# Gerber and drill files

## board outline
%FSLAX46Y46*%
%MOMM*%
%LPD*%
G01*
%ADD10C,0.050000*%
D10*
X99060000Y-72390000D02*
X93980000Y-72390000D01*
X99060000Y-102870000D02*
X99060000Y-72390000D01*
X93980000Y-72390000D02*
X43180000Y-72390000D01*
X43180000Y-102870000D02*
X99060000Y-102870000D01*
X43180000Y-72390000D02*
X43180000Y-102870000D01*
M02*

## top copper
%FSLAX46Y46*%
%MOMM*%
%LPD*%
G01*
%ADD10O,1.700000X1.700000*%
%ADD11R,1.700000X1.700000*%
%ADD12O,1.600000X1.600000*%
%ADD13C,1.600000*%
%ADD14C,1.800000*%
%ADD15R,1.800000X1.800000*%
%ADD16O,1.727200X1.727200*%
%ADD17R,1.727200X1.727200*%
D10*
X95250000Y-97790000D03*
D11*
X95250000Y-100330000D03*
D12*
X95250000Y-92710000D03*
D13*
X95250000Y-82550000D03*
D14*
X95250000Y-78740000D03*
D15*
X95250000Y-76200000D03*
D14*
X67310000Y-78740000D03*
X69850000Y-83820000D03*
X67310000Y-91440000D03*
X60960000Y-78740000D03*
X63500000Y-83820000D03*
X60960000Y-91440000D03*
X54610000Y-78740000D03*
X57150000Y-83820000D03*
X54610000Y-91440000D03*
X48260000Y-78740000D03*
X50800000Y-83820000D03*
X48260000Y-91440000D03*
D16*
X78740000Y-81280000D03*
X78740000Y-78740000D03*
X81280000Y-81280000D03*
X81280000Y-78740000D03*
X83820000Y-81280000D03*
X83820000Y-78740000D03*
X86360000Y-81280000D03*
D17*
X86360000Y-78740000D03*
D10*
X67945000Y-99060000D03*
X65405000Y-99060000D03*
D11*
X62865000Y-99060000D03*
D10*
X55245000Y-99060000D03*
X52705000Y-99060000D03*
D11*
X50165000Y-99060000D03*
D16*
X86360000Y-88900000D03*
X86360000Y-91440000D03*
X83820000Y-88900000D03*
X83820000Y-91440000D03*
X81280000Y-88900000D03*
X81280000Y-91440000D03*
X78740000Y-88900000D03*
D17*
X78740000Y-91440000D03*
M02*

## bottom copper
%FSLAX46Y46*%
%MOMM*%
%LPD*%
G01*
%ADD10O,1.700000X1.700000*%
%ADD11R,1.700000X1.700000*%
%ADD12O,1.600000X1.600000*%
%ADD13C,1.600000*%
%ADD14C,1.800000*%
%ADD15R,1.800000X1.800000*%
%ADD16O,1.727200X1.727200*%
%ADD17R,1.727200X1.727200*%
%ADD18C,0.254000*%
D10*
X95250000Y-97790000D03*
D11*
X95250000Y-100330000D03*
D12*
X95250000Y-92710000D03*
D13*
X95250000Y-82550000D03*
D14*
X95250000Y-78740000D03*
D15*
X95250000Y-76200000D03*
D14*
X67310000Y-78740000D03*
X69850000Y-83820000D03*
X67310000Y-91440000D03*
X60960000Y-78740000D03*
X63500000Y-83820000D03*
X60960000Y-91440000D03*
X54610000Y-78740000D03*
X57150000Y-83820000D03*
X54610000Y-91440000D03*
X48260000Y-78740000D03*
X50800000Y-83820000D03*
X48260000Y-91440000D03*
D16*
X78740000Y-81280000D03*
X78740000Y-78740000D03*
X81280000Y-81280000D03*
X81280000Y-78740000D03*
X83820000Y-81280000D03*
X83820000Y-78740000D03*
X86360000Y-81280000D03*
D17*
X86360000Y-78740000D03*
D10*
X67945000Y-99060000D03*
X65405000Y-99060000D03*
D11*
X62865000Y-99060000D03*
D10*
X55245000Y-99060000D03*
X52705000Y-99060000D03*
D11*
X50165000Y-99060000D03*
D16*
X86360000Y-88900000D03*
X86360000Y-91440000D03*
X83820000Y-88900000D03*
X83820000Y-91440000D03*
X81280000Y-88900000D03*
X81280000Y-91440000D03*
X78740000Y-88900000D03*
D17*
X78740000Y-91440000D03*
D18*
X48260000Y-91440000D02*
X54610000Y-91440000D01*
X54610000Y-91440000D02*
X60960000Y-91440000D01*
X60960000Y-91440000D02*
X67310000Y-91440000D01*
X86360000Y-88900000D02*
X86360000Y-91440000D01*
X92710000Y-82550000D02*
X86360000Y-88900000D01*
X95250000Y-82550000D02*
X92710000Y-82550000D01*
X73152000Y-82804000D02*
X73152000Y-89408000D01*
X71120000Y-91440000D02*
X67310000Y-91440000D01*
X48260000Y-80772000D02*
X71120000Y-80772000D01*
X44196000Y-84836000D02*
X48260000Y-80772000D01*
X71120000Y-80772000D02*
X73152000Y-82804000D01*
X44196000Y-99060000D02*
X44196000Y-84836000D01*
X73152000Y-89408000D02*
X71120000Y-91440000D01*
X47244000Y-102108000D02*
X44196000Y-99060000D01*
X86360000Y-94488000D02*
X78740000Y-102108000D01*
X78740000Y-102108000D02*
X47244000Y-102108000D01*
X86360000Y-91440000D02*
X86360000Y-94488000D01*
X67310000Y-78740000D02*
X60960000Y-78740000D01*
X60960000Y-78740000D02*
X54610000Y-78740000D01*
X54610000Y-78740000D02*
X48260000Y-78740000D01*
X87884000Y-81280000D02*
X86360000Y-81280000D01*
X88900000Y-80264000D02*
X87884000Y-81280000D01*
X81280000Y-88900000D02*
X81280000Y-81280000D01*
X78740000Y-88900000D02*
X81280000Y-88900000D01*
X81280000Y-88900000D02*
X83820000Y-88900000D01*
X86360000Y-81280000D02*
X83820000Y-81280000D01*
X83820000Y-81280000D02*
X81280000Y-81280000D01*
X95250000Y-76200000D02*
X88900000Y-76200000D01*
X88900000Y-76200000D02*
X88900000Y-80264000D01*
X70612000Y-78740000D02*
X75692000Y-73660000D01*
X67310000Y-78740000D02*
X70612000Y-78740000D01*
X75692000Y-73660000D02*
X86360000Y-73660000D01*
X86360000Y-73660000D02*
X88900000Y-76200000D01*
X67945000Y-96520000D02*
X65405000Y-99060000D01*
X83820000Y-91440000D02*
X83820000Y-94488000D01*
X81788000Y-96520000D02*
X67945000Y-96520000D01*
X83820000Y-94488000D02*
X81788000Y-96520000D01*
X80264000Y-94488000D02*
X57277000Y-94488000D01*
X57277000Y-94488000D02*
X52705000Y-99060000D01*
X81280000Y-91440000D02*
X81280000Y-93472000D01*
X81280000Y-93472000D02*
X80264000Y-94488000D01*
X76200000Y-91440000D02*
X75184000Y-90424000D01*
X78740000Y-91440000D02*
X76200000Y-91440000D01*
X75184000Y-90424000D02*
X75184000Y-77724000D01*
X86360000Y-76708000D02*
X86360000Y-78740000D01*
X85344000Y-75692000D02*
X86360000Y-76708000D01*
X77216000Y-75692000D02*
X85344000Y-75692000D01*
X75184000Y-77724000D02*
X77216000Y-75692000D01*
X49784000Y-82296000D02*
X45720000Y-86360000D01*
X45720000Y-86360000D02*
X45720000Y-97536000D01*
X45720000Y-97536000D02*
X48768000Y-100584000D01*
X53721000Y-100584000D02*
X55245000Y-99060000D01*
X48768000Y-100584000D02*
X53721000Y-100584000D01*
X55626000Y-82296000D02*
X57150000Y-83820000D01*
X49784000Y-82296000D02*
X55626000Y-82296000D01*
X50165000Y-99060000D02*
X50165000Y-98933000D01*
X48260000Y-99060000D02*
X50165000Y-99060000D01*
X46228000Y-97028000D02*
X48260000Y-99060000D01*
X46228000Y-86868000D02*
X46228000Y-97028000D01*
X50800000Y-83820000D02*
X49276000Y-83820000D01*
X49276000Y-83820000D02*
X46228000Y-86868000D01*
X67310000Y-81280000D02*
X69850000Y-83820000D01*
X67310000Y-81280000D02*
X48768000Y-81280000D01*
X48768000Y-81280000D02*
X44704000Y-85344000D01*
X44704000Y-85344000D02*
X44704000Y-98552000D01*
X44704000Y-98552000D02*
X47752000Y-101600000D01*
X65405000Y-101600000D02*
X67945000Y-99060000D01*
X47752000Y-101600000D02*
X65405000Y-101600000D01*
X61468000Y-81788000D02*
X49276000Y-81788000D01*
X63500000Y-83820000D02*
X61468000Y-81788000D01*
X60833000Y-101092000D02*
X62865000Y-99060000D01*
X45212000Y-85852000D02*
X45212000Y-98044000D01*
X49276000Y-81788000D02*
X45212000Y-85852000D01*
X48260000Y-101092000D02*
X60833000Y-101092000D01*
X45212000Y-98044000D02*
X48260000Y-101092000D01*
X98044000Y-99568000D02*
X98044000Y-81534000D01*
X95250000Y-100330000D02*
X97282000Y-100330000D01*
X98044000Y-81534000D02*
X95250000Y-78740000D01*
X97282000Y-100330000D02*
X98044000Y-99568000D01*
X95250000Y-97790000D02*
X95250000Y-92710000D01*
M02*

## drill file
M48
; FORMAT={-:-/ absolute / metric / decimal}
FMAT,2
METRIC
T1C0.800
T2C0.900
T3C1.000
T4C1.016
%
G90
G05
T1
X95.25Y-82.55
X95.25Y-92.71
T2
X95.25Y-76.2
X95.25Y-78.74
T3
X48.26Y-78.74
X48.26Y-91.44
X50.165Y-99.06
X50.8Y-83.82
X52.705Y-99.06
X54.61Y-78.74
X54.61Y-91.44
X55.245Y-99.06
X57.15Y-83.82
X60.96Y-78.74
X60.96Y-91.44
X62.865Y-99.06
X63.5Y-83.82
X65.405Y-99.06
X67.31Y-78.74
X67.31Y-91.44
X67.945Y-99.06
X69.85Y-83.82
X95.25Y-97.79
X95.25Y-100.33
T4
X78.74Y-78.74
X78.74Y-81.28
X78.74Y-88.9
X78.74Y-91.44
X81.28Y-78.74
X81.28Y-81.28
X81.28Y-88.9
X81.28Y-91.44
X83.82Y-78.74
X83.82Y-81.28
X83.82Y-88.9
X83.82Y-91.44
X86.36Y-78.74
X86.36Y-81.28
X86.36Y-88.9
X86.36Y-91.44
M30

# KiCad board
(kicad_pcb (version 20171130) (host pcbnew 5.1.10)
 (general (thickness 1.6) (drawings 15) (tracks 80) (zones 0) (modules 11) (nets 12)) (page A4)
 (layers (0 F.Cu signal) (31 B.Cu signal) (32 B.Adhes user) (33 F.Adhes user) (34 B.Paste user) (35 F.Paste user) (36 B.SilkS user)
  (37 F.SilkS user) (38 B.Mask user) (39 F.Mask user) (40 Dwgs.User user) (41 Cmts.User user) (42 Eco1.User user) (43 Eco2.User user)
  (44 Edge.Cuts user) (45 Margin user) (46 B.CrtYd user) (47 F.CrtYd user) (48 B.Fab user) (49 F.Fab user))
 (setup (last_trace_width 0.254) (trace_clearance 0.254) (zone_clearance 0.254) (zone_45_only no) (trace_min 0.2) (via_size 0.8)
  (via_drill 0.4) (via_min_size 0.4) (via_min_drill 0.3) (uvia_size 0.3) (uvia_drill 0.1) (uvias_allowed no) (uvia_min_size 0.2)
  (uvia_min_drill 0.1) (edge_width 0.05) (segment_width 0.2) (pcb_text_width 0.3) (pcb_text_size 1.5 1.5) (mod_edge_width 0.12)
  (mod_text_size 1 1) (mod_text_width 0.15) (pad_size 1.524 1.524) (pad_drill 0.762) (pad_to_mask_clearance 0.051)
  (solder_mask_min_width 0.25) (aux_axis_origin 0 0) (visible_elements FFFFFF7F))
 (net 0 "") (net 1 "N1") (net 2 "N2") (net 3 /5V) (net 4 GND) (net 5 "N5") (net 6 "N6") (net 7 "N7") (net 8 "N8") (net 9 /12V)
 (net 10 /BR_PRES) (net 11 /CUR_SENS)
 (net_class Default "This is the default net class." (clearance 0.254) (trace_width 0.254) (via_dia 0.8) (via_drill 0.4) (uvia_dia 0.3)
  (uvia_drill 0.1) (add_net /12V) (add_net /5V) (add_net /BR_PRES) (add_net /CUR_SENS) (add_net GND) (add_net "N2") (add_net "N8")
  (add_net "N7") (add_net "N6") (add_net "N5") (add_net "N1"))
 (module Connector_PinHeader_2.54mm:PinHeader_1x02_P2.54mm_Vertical (layer F.Cu) (at 95.25 100.33 180)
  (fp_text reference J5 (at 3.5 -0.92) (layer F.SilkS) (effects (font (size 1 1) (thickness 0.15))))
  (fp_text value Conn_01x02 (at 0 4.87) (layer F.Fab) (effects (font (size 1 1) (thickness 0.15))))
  (pad 2 thru_hole oval (at 0 2.54 180) (size 1.7 1.7) (drill 1) (layers *.Cu *.Mask) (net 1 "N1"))
  (pad 1 thru_hole rect (at 0 0 180) (size 1.7 1.7) (drill 1) (layers *.Cu *.Mask) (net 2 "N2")))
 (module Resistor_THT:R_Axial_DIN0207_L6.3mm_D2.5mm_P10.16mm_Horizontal (layer F.Cu) (at 95.25 82.55 270)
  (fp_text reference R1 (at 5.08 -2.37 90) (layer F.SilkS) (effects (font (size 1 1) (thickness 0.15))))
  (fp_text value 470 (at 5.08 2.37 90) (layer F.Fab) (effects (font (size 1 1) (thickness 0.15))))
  (pad 2 thru_hole oval (at 10.16 0 270) (size 1.6 1.6) (drill 0.8) (layers *.Cu *.Mask) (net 1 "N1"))
  (pad 1 thru_hole circle (at 0 0 270) (size 1.6 1.6) (drill 0.8) (layers *.Cu *.Mask) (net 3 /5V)))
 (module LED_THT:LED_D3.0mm (layer F.Cu) (at 95.25 76.2 270)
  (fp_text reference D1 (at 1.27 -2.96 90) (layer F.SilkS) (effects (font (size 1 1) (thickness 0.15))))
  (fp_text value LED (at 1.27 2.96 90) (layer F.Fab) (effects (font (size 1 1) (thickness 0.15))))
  (pad 2 thru_hole circle (at 2.54 0 270) (size 1.8 1.8) (drill 0.9) (layers *.Cu *.Mask) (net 2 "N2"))
  (pad 1 thru_hole rect (at 0 0 270) (size 1.8 1.8) (drill 0.9) (layers *.Cu *.Mask) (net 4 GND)))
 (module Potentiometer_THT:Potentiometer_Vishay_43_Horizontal (layer F.Cu) (at 67.31 91.44 270)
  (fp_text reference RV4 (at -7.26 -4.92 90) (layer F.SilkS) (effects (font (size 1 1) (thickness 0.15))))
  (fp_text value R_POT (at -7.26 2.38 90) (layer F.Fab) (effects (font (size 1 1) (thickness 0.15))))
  (pad 3 thru_hole circle (at -12.7 0 270) (size 1.8 1.8) (drill 1) (layers *.Cu *.Mask) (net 4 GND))
  (pad 2 thru_hole circle (at -7.62 -2.54 270) (size 1.8 1.8) (drill 1) (layers *.Cu *.Mask) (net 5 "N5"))
  (pad 1 thru_hole circle (at 0 0 270) (size 1.8 1.8) (drill 1) (layers *.Cu *.Mask) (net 3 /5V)))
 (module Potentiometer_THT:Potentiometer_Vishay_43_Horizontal (layer F.Cu) (at 60.96 91.44 270)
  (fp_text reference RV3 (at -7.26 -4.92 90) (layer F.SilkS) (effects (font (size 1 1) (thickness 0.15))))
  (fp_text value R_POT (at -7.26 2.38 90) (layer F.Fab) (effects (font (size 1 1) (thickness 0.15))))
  (pad 3 thru_hole circle (at -12.7 0 270) (size 1.8 1.8) (drill 1) (layers *.Cu *.Mask) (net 4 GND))
  (pad 2 thru_hole circle (at -7.62 -2.54 270) (size 1.8 1.8) (drill 1) (layers *.Cu *.Mask) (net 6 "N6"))
  (pad 1 thru_hole circle (at 0 0 270) (size 1.8 1.8) (drill 1) (layers *.Cu *.Mask) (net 3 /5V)))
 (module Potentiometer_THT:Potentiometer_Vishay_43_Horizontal (layer F.Cu) (at 54.61 91.44 270)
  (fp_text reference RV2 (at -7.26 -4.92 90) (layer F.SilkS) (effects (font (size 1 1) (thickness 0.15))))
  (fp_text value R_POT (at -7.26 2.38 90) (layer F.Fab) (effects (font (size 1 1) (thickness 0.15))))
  (pad 3 thru_hole circle (at -12.7 0 270) (size 1.8 1.8) (drill 1) (layers *.Cu *.Mask) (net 4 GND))
  (pad 2 thru_hole circle (at -7.62 -2.54 270) (size 1.8 1.8) (drill 1) (layers *.Cu *.Mask) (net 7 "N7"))
  (pad 1 thru_hole circle (at 0 0 270) (size 1.8 1.8) (drill 1) (layers *.Cu *.Mask) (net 3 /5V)))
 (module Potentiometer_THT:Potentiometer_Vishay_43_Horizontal (layer F.Cu) (at 48.26 91.44 270)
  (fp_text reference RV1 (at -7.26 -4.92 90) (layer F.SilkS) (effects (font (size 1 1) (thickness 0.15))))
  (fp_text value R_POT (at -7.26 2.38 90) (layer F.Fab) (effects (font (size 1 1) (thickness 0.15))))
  (pad 3 thru_hole circle (at -12.7 0 270) (size 1.8 1.8) (drill 1) (layers *.Cu *.Mask) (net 4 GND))
  (pad 2 thru_hole circle (at -7.62 -2.54 270) (size 1.8 1.8) (drill 1) (layers *.Cu *.Mask) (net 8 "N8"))
  (pad 1 thru_hole circle (at 0 0 270) (size 1.8 1.8) (drill 1) (layers *.Cu *.Mask) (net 3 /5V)))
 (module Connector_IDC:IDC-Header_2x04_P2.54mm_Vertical (layer F.Cu) (at 86.36 78.74 270)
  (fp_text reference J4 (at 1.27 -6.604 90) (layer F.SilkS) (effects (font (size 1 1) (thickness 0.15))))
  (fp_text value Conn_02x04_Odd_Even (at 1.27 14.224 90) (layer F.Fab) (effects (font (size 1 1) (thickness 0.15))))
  (pad 8 thru_hole oval (at 2.54 7.62 270) (size 1.7272 1.7272) (drill 1.016) (layers *.Cu *.Mask))
  (pad 7 thru_hole oval (at 0 7.62 270) (size 1.7272 1.7272) (drill 1.016) (layers *.Cu *.Mask))
  (pad 6 thru_hole oval (at 2.54 5.08 270) (size 1.7272 1.7272) (drill 1.016) (layers *.Cu *.Mask) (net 4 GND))
  (pad 5 thru_hole oval (at 0 5.08 270) (size 1.7272 1.7272) (drill 1.016) (layers *.Cu *.Mask))
  (pad 4 thru_hole oval (at 2.54 2.54 270) (size 1.7272 1.7272) (drill 1.016) (layers *.Cu *.Mask) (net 4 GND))
  (pad 3 thru_hole oval (at 0 2.54 270) (size 1.7272 1.7272) (drill 1.016) (layers *.Cu *.Mask))
  (pad 2 thru_hole oval (at 2.54 0 270) (size 1.7272 1.7272) (drill 1.016) (layers *.Cu *.Mask) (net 4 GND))
  (pad 1 thru_hole rect (at 0 0 270) (size 1.7272 1.7272) (drill 1.016) (layers *.Cu *.Mask) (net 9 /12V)))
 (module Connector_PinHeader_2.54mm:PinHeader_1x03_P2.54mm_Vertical (layer F.Cu) (at 62.865 99.06 90)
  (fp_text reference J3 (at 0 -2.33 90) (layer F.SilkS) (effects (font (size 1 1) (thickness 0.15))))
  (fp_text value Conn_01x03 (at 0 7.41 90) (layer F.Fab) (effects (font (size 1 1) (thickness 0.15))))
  (pad 3 thru_hole oval (at 0 5.08 90) (size 1.7 1.7) (drill 1) (layers *.Cu *.Mask) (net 5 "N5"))
  (pad 2 thru_hole oval (at 0 2.54 90) (size 1.7 1.7) (drill 1) (layers *.Cu *.Mask) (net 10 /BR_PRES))
  (pad 1 thru_hole rect (at 0 0 90) (size 1.7 1.7) (drill 1) (layers *.Cu *.Mask) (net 6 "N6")))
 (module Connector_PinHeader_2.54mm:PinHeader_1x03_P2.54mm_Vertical (layer F.Cu) (at 50.165 99.06 90)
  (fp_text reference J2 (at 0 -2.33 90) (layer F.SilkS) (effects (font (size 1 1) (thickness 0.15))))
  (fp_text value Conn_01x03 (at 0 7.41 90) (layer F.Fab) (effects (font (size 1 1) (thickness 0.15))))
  (pad 3 thru_hole oval (at 0 5.08 90) (size 1.7 1.7) (drill 1) (layers *.Cu *.Mask) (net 7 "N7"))
  (pad 2 thru_hole oval (at 0 2.54 90) (size 1.7 1.7) (drill 1) (layers *.Cu *.Mask) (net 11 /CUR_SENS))
  (pad 1 thru_hole rect (at 0 0 90) (size 1.7 1.7) (drill 1) (layers *.Cu *.Mask) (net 8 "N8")))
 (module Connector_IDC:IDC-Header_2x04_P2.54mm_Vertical (layer F.Cu) (at 78.74 91.44 90)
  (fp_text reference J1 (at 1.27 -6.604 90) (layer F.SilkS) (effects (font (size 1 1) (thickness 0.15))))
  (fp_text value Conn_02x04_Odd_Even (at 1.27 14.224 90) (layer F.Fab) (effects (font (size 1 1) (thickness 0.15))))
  (pad 8 thru_hole oval (at 2.54 7.62 90) (size 1.7272 1.7272) (drill 1.016) (layers *.Cu *.Mask) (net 3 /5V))
  (pad 7 thru_hole oval (at 0 7.62 90) (size 1.7272 1.7272) (drill 1.016) (layers *.Cu *.Mask) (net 3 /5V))
  (pad 6 thru_hole oval (at 2.54 5.08 90) (size 1.7272 1.7272) (drill 1.016) (layers *.Cu *.Mask) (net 4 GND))
  (pad 5 thru_hole oval (at 0 5.08 90) (size 1.7272 1.7272) (drill 1.016) (layers *.Cu *.Mask) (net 10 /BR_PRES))
  (pad 4 thru_hole oval (at 2.54 2.54 90) (size 1.7272 1.7272) (drill 1.016) (layers *.Cu *.Mask) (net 4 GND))
  (pad 3 thru_hole oval (at 0 2.54 90) (size 1.7272 1.7272) (drill 1.016) (layers *.Cu *.Mask) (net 11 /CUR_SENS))
  (pad 2 thru_hole oval (at 2.54 0 90) (size 1.7272 1.7272) (drill 1.016) (layers *.Cu *.Mask) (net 4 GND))
  (pad 1 thru_hole rect (at 0 0 90) (size 1.7272 1.7272) (drill 1.016) (layers *.Cu *.Mask) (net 9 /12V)))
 (gr_line (start 99.06 72.39) (end 93.98 72.39) (layer Edge.Cuts) (width 0.05))
 (gr_line (start 99.06 102.87) (end 99.06 72.39) (layer Edge.Cuts) (width 0.05))
 (gr_line (start 93.98 72.39) (end 43.18 72.39) (layer Edge.Cuts) (width 0.05))
 (gr_line (start 43.18 102.87) (end 99.06 102.87) (layer Edge.Cuts) (width 0.05))
 (gr_line (start 43.18 72.39) (end 43.18 102.87) (layer Edge.Cuts) (width 0.05))
 (segment (start 48.26 91.44) (end 54.61 91.44) (width 0.254) (layer B.Cu) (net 3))
 (segment (start 54.61 91.44) (end 60.96 91.44) (width 0.254) (layer B.Cu) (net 3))
 (segment (start 60.96 91.44) (end 67.31 91.44) (width 0.254) (layer B.Cu) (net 3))
 (segment (start 86.36 88.9) (end 86.36 91.44) (width 0.254) (layer B.Cu) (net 3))
 (segment (start 92.71 82.55) (end 86.36 88.9) (width 0.254) (layer B.Cu) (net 3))
 (segment (start 95.25 82.55) (end 92.71 82.55) (width 0.254) (layer B.Cu) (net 3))
 (segment (start 73.152 82.804) (end 73.152 89.408) (width 0.254) (layer B.Cu) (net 3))
 (segment (start 71.12 91.44) (end 67.31 91.44) (width 0.254) (layer B.Cu) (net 3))
 (segment (start 48.26 80.772) (end 71.12 80.772) (width 0.254) (layer B.Cu) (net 3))
 (segment (start 44.196 84.836) (end 48.26 80.772) (width 0.254) (layer B.Cu) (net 3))
 (segment (start 71.12 80.772) (end 73.152 82.804) (width 0.254) (layer B.Cu) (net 3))
 (segment (start 44.196 99.06) (end 44.196 84.836) (width 0.254) (layer B.Cu) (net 3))
 (segment (start 73.152 89.408) (end 71.12 91.44) (width 0.254) (layer B.Cu) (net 3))
 (segment (start 47.244 102.108) (end 44.196 99.06) (width 0.254) (layer B.Cu) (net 3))
 (segment (start 86.36 94.488) (end 78.74 102.108) (width 0.254) (layer B.Cu) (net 3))
 (segment (start 78.74 102.108) (end 47.244 102.108) (width 0.254) (layer B.Cu) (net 3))
 (segment (start 86.36 91.44) (end 86.36 94.488) (width 0.254) (layer B.Cu) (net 3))
 (segment (start 67.31 78.74) (end 60.96 78.74) (width 0.254) (layer B.Cu) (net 4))
 (segment (start 60.96 78.74) (end 54.61 78.74) (width 0.254) (layer B.Cu) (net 4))
 (segment (start 54.61 78.74) (end 48.26 78.74) (width 0.254) (layer B.Cu) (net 4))
 (segment (start 87.884 81.28) (end 86.36 81.28) (width 0.254) (layer B.Cu) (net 4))
 (segment (start 88.9 80.264) (end 87.884 81.28) (width 0.254) (layer B.Cu) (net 4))
 (segment (start 81.28 88.9) (end 81.28 81.28) (width 0.254) (layer B.Cu) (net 4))
 (segment (start 78.74 88.9) (end 81.28 88.9) (width 0.254) (layer B.Cu) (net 4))
 (segment (start 81.28 88.9) (end 83.82 88.9) (width 0.254) (layer B.Cu) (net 4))
 (segment (start 86.36 81.28) (end 83.82 81.28) (width 0.254) (layer B.Cu) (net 4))
 (segment (start 83.82 81.28) (end 81.28 81.28) (width 0.254) (layer B.Cu) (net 4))
 (segment (start 95.25 76.2) (end 88.9 76.2) (width 0.254) (layer B.Cu) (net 4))
 (segment (start 88.9 76.2) (end 88.9 80.264) (width 0.254) (layer B.Cu) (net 4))
 (segment (start 70.612 78.74) (end 75.692 73.66) (width 0.254) (layer B.Cu) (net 4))
 (segment (start 67.31 78.74) (end 70.612 78.74) (width 0.254) (layer B.Cu) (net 4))
 (segment (start 75.692 73.66) (end 86.36 73.66) (width 0.254) (layer B.Cu) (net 4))
 (segment (start 86.36 73.66) (end 88.9 76.2) (width 0.254) (layer B.Cu) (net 4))
 (segment (start 67.945 96.52) (end 65.405 99.06) (width 0.254) (layer B.Cu) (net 10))
 (segment (start 83.82 91.44) (end 83.82 94.488) (width 0.254) (layer B.Cu) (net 10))
 (segment (start 81.788 96.52) (end 67.945 96.52) (width 0.254) (layer B.Cu) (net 10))
 (segment (start 83.82 94.488) (end 81.788 96.52) (width 0.254) (layer B.Cu) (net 10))
 (segment (start 80.264 94.488) (end 57.277 94.488) (width 0.254) (layer B.Cu) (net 11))
 (segment (start 57.277 94.488) (end 52.705 99.06) (width 0.254) (layer B.Cu) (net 11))
 (segment (start 81.28 91.44) (end 81.28 93.472) (width 0.254) (layer B.Cu) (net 11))
 (segment (start 81.28 93.472) (end 80.264 94.488) (width 0.254) (layer B.Cu) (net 11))
 (segment (start 76.2 91.44) (end 75.184 90.424) (width 0.254) (layer B.Cu) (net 9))
 (segment (start 78.74 91.44) (end 76.2 91.44) (width 0.254) (layer B.Cu) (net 9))
 (segment (start 75.184 90.424) (end 75.184 77.724) (width 0.254) (layer B.Cu) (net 9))
 (segment (start 86.36 76.708) (end 86.36 78.74) (width 0.254) (layer B.Cu) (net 9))
 (segment (start 85.344 75.692) (end 86.36 76.708) (width 0.254) (layer B.Cu) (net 9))
 (segment (start 77.216 75.692) (end 85.344 75.692) (width 0.254) (layer B.Cu) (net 9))
 (segment (start 75.184 77.724) (end 77.216 75.692) (width 0.254) (layer B.Cu) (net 9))
 (segment (start 49.784 82.296) (end 45.72 86.36) (width 0.254) (layer B.Cu) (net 7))
 (segment (start 45.72 86.36) (end 45.72 97.536) (width 0.254) (layer B.Cu) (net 7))
 (segment (start 45.72 97.536) (end 48.768 100.584) (width 0.254) (layer B.Cu) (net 7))
 (segment (start 53.721 100.584) (end 55.245 99.06) (width 0.254) (layer B.Cu) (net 7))
 (segment (start 48.768 100.584) (end 53.721 100.584) (width 0.254) (layer B.Cu) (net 7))
 (segment (start 55.626 82.296) (end 57.15 83.82) (width 0.254) (layer B.Cu) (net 7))
 (segment (start 49.784 82.296) (end 55.626 82.296) (width 0.254) (layer B.Cu) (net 7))
 (segment (start 50.165 99.06) (end 50.165 98.933) (width 0.254) (layer B.Cu) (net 8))
 (segment (start 48.26 99.06) (end 50.165 99.06) (width 0.254) (layer B.Cu) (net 8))
 (segment (start 46.228 97.028) (end 48.26 99.06) (width 0.254) (layer B.Cu) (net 8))
 (segment (start 46.228 86.868) (end 46.228 97.028) (width 0.254) (layer B.Cu) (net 8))
 (segment (start 50.8 83.82) (end 49.276 83.82) (width 0.254) (layer B.Cu) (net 8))
 (segment (start 49.276 83.82) (end 46.228 86.868) (width 0.254) (layer B.Cu) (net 8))
 (segment (start 67.31 81.28) (end 69.85 83.82) (width 0.254) (layer B.Cu) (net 5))
 (segment (start 67.31 81.28) (end 48.768 81.28) (width 0.254) (layer B.Cu) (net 5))
 (segment (start 48.768 81.28) (end 44.704 85.344) (width 0.254) (layer B.Cu) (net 5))
 (segment (start 44.704 85.344) (end 44.704 98.552) (width 0.254) (layer B.Cu) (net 5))
 (segment (start 44.704 98.552) (end 47.752 101.6) (width 0.254) (layer B.Cu) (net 5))
 (segment (start 65.405 101.6) (end 67.945 99.06) (width 0.254) (layer B.Cu) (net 5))
 (segment (start 47.752 101.6) (end 65.405 101.6) (width 0.254) (layer B.Cu) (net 5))
 (segment (start 61.468 81.788) (end 49.276 81.788) (width 0.254) (layer B.Cu) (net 6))
 (segment (start 63.5 83.82) (end 61.468 81.788) (width 0.254) (layer B.Cu) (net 6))
 (segment (start 60.833 101.092) (end 62.865 99.06) (width 0.254) (layer B.Cu) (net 6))
 (segment (start 45.212 85.852) (end 45.212 98.044) (width 0.254) (layer B.Cu) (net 6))
 (segment (start 49.276 81.788) (end 45.212 85.852) (width 0.254) (layer B.Cu) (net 6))
 (segment (start 48.26 101.092) (end 60.833 101.092) (width 0.254) (layer B.Cu) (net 6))
 (segment (start 45.212 98.044) (end 48.26 101.092) (width 0.254) (layer B.Cu) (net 6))
 (segment (start 98.044 99.568) (end 98.044 81.534) (width 0.254) (layer B.Cu) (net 2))
 (segment (start 95.25 100.33) (end 97.282 100.33) (width 0.254) (layer B.Cu) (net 2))
 (segment (start 98.044 81.534) (end 95.25 78.74) (width 0.254) (layer B.Cu) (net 2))
 (segment (start 97.282 100.33) (end 98.044 99.568) (width 0.254) (layer B.Cu) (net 2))
 (segment (start 95.25 97.79) (end 95.25 92.71) (width 0.254) (layer B.Cu) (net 1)))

